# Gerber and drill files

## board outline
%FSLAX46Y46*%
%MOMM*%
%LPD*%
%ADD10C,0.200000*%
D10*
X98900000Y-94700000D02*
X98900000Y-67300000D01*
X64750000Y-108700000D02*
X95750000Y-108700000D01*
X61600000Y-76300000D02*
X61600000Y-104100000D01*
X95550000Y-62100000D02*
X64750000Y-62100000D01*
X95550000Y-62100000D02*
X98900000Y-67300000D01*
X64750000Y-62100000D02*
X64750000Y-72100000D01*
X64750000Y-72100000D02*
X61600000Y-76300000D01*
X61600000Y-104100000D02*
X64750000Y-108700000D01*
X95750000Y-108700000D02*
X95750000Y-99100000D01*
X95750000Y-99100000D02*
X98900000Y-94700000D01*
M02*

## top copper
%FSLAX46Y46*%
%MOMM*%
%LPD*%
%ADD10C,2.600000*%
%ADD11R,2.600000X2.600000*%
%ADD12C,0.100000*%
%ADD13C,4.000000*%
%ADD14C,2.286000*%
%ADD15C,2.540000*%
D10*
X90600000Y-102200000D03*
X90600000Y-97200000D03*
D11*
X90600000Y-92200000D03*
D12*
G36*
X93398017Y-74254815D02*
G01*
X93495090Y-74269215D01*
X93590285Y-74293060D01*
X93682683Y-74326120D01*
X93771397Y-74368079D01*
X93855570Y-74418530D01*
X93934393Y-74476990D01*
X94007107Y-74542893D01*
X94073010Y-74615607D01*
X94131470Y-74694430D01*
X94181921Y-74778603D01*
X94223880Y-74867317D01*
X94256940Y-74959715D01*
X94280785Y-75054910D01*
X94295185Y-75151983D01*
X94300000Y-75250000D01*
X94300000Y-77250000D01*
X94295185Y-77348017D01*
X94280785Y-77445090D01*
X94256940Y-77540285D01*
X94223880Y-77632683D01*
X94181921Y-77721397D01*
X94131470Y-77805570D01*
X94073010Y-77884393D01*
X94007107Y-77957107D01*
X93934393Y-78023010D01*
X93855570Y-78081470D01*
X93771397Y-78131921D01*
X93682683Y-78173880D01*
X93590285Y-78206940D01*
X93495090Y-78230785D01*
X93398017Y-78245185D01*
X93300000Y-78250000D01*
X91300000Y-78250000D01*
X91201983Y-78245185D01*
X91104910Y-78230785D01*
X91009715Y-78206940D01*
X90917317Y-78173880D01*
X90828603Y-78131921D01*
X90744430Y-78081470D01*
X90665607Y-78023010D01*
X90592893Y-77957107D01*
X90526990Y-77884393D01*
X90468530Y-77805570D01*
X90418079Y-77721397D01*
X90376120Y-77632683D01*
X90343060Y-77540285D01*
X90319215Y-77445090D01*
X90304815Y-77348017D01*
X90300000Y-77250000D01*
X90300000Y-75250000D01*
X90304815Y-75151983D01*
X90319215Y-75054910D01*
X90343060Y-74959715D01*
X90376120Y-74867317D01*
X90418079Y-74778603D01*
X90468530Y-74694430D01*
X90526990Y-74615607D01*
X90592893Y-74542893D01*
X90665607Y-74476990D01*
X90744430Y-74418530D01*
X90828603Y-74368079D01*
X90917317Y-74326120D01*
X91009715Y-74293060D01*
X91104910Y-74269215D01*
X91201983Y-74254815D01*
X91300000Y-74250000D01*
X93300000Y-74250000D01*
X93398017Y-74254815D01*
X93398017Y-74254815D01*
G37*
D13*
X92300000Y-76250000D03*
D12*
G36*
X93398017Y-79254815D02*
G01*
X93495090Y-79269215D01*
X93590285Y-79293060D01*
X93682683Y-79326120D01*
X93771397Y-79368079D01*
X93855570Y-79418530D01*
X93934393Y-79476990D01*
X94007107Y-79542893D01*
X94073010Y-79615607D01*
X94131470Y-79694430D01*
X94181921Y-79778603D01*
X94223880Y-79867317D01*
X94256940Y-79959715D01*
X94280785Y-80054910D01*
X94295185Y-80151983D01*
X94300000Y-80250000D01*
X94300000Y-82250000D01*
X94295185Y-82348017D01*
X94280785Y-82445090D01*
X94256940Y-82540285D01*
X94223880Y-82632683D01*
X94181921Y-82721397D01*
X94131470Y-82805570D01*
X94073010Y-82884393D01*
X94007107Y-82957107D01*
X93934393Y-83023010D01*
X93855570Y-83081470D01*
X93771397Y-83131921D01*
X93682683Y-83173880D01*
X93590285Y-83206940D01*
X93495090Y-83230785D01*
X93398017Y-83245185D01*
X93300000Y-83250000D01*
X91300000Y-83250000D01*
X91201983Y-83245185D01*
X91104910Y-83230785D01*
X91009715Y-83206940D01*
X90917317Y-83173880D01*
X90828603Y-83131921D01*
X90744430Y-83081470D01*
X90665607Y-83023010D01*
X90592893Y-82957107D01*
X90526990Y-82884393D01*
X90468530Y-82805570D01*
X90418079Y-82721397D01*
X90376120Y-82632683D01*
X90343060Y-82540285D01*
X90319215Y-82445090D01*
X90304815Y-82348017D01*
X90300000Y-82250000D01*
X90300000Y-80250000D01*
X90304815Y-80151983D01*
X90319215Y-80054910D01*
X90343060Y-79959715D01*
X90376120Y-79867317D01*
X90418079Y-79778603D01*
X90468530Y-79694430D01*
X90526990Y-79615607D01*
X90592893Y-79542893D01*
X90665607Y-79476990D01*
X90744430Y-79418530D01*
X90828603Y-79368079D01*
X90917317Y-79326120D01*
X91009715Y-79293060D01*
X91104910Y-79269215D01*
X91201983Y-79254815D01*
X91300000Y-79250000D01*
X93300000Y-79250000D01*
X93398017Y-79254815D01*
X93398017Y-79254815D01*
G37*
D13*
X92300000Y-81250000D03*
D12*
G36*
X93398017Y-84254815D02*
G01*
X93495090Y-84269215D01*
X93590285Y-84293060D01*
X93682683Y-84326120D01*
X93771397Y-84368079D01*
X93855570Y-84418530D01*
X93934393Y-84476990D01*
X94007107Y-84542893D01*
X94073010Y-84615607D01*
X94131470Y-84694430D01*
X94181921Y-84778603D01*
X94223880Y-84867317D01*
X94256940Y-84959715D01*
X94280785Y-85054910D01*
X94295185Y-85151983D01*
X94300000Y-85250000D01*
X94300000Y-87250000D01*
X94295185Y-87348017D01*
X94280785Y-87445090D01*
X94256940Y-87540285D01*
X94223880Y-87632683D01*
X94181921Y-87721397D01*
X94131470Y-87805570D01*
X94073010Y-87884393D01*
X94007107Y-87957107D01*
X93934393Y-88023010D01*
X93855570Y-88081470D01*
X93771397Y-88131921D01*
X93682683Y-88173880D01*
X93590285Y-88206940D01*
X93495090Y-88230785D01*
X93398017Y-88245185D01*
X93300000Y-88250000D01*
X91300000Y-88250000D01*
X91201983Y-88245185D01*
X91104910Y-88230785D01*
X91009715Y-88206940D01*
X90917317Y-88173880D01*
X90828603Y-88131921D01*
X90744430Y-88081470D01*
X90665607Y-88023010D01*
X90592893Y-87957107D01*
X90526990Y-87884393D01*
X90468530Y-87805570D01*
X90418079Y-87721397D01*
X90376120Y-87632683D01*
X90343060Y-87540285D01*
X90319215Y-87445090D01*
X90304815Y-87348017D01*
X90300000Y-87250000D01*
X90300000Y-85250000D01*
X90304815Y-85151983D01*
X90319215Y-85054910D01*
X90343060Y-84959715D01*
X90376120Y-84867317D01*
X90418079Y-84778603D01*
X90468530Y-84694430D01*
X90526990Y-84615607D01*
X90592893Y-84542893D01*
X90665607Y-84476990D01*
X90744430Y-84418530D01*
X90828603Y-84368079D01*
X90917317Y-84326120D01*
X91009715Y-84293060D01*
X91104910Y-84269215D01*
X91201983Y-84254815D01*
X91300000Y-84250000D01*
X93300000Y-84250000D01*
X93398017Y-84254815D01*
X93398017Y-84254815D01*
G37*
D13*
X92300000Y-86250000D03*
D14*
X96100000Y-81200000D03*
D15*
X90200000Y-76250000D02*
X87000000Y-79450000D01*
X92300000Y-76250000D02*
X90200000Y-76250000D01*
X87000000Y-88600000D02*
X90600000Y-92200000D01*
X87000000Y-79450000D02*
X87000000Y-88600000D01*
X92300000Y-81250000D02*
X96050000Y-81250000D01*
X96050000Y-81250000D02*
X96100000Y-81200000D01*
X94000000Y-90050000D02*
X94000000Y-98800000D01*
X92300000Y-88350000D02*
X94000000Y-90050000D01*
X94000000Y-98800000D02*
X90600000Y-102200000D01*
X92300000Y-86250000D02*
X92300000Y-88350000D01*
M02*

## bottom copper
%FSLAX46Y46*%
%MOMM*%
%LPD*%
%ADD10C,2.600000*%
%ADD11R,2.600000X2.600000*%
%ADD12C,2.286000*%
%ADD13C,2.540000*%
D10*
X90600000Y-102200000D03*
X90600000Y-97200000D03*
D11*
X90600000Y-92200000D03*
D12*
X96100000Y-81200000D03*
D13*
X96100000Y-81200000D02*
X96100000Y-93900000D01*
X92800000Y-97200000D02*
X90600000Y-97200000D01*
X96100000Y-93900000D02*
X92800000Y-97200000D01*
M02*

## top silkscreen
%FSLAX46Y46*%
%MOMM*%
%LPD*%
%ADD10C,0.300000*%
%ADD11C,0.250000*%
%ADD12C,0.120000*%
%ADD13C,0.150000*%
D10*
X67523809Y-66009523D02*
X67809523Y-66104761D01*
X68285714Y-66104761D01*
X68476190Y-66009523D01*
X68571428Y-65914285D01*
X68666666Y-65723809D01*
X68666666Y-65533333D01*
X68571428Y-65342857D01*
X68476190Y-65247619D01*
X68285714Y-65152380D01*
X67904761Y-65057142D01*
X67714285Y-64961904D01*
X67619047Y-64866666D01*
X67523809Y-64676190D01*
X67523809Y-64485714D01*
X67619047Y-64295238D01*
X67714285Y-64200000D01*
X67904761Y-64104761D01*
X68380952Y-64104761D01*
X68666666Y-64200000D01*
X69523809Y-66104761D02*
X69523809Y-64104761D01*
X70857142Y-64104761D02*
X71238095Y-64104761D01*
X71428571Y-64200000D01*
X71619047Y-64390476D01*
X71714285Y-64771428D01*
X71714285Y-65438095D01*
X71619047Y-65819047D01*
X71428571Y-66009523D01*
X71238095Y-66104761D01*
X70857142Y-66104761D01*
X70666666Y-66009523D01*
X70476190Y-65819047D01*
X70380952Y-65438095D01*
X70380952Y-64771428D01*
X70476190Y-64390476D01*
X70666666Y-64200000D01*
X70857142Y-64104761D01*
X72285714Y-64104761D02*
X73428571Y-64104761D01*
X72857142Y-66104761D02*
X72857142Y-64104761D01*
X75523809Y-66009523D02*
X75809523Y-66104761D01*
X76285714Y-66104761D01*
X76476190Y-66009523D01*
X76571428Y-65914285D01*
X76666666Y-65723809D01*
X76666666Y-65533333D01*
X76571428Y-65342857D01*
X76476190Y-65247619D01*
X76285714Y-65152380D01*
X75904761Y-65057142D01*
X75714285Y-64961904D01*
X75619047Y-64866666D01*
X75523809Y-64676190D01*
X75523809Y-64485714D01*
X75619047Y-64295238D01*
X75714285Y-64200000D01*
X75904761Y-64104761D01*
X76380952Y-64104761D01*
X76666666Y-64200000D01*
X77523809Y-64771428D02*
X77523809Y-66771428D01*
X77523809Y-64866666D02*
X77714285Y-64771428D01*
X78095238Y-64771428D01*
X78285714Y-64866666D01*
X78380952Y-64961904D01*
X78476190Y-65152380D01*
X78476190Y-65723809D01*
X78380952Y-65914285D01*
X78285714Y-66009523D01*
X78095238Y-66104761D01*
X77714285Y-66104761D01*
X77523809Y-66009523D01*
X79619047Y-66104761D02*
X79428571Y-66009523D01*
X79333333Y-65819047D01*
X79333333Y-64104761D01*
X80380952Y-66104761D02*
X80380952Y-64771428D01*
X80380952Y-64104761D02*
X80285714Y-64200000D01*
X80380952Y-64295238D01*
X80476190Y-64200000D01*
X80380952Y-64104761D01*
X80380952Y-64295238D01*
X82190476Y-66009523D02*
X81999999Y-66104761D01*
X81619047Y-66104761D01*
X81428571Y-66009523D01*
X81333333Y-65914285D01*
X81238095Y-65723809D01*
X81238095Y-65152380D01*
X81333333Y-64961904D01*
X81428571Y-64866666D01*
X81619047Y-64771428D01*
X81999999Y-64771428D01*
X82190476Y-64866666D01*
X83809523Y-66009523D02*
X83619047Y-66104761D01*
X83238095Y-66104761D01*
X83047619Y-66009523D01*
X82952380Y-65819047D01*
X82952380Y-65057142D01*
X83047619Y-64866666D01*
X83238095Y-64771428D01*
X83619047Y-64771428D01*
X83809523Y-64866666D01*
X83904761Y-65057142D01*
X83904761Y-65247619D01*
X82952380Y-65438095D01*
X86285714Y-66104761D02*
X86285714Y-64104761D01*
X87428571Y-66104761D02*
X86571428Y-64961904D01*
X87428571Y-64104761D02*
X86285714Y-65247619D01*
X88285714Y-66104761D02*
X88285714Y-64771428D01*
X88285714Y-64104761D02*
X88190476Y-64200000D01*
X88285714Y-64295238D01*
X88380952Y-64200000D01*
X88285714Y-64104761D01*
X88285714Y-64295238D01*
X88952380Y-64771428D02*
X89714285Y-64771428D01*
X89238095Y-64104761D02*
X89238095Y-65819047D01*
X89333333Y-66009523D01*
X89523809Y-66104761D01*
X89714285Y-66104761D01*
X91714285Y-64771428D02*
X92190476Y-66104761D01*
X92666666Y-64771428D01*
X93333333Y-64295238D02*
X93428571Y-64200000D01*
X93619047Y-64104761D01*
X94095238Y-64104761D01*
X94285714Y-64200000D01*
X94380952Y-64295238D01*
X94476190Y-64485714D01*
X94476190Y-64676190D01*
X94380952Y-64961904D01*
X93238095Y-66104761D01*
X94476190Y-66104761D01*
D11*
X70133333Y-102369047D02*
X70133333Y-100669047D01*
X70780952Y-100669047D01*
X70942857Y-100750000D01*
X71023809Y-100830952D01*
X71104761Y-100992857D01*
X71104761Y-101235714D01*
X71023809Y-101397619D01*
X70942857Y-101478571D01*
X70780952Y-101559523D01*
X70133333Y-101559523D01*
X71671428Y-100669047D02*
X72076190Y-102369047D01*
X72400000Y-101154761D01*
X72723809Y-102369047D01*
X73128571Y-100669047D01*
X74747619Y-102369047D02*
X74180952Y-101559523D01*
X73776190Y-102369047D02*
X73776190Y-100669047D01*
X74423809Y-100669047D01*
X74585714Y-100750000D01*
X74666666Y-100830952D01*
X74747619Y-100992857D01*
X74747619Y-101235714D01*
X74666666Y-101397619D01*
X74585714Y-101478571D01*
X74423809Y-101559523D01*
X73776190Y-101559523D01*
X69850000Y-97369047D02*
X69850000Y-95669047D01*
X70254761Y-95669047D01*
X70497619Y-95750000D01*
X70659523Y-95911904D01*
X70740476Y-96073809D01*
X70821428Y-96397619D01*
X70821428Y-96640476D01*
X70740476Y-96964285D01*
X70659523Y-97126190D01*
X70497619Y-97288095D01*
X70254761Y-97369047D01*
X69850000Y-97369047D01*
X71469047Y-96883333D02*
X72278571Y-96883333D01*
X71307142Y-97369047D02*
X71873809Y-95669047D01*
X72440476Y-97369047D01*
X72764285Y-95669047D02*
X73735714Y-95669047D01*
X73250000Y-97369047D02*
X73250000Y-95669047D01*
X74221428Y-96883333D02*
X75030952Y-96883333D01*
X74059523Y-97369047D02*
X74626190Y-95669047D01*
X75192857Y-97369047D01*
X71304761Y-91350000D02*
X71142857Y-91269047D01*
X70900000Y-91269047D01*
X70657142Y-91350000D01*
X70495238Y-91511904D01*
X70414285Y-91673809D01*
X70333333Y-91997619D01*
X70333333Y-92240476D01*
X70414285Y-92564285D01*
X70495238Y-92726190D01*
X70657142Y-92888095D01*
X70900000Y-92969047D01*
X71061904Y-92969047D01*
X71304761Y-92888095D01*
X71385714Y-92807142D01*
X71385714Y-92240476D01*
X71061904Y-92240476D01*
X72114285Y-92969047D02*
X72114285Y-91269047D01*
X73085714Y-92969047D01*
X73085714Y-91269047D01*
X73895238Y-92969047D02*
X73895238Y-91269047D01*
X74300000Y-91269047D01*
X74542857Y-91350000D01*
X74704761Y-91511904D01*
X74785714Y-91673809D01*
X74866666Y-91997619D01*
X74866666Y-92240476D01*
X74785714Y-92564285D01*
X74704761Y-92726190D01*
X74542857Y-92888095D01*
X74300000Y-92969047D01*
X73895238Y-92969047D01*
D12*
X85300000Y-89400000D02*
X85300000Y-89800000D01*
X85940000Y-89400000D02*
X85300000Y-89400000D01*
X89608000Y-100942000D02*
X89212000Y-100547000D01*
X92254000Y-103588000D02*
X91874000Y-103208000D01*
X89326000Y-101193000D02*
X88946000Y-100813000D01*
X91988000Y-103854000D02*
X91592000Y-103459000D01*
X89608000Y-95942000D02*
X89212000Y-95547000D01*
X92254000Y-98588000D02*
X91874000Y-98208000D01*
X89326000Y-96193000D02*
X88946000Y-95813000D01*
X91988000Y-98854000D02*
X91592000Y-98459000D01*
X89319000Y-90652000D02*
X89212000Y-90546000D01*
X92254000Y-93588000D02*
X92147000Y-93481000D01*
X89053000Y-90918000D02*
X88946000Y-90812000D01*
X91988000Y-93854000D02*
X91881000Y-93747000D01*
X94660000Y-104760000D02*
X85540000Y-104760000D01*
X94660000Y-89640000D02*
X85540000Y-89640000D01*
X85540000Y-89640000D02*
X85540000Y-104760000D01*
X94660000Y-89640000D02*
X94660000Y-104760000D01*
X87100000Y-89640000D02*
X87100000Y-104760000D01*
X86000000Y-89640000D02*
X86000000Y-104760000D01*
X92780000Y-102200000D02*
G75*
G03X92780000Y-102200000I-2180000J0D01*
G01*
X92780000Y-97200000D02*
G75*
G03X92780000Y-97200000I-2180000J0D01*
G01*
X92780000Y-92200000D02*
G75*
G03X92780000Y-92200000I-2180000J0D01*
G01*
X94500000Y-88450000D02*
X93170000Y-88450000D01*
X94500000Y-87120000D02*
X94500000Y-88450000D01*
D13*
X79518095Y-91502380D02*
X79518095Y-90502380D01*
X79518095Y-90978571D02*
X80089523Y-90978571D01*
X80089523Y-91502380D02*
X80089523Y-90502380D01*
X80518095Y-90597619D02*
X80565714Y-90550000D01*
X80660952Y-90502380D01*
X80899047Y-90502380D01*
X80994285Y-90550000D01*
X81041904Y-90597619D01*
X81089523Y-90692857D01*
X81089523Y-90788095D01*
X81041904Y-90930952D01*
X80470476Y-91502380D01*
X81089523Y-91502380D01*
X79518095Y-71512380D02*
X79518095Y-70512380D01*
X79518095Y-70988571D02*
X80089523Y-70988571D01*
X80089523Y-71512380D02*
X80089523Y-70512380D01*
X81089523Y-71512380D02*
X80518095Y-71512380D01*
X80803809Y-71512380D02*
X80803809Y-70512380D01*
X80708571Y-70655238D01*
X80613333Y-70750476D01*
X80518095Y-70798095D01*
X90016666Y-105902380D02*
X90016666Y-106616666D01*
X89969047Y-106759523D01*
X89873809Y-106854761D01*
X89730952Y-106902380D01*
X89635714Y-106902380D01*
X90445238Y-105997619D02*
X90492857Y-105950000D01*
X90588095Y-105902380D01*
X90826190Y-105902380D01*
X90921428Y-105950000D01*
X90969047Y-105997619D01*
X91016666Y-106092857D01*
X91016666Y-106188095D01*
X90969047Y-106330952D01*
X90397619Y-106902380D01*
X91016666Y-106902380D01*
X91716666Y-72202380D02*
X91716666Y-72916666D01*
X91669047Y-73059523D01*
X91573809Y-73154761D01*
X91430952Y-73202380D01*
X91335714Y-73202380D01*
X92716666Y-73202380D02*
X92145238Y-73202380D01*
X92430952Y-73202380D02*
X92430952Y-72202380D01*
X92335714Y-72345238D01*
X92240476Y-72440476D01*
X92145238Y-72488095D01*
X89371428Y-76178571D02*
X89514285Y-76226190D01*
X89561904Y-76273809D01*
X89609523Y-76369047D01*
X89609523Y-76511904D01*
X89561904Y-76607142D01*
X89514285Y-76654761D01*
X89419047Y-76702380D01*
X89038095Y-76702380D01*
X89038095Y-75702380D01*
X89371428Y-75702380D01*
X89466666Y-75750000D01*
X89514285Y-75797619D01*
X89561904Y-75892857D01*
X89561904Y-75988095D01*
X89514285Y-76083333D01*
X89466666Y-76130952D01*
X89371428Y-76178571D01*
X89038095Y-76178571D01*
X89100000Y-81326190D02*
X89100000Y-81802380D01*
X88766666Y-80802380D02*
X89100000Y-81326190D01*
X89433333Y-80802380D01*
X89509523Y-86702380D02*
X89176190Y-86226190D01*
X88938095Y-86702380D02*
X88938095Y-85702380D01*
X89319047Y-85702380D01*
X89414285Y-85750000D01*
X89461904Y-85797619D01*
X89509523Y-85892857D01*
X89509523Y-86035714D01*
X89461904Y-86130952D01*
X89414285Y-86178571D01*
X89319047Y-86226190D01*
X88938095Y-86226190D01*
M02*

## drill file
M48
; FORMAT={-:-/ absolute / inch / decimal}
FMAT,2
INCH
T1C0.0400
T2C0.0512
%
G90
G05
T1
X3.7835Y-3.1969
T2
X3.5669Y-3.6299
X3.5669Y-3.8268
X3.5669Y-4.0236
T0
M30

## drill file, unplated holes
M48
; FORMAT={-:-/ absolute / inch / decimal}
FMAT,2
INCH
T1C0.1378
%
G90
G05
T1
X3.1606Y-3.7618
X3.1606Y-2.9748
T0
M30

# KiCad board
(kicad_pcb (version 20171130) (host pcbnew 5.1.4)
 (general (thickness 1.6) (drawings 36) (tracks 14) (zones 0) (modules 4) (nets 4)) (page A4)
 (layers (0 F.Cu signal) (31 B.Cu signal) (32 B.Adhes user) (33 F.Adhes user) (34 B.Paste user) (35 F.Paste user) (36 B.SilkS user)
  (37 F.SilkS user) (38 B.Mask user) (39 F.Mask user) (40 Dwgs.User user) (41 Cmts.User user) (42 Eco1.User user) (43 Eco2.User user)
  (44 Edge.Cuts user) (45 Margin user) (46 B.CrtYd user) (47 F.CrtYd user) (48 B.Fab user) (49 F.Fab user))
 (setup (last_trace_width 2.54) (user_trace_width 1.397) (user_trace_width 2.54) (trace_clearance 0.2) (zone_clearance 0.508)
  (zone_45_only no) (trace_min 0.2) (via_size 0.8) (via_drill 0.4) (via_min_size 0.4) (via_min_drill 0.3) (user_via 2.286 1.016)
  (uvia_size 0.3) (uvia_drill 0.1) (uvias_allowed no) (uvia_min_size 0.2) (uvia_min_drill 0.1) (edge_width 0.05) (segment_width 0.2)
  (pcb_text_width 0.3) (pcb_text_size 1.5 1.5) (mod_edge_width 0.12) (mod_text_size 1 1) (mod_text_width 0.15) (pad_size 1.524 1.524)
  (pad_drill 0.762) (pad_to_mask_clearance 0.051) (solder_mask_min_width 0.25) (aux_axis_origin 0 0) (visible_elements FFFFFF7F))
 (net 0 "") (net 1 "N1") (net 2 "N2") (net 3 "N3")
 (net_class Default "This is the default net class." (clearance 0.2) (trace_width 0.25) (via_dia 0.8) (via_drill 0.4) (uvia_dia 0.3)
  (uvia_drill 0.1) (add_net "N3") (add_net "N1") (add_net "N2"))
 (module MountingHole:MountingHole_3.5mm (layer F.Cu) (at 80.28 95.55)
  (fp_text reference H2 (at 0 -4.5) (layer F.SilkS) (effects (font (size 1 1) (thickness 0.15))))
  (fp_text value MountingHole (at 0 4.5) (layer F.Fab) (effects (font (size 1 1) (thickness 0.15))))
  (pad 1 np_thru_hole circle (at 0 0) (size 3.5 3.5) (drill 3.5) (layers *.Cu *.Mask)))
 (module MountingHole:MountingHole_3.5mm (layer F.Cu) (at 80.28 75.56)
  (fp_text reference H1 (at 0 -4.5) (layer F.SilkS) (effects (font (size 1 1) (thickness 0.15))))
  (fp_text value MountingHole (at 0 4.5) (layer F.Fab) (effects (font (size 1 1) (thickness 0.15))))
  (pad 1 np_thru_hole circle (at 0 0) (size 3.5 3.5) (drill 3.5) (layers *.Cu *.Mask)))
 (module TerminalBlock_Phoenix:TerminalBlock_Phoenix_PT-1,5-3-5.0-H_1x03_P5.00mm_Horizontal (layer F.Cu) (at 90.6 92.2 270)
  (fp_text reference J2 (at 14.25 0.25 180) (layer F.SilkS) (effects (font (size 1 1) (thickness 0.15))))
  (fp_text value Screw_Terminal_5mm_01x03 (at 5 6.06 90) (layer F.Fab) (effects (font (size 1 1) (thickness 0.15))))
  (fp_line (start -2.8 5.3) (end -2.4 5.3) (layer F.SilkS) (width 0.12))
  (fp_line (start -2.8 4.66) (end -2.8 5.3) (layer F.SilkS) (width 0.12))
  (fp_line (start 8.742 0.992) (end 8.347 1.388) (layer F.SilkS) (width 0.12))
  (fp_line (start 11.388 -1.654) (end 11.008 -1.274) (layer F.SilkS) (width 0.12))
  (fp_line (start 8.993 1.274) (end 8.613 1.654) (layer F.SilkS) (width 0.12))
  (fp_line (start 11.654 -1.388) (end 11.259 -0.992) (layer F.SilkS) (width 0.12))
  (fp_line (start 3.742 0.992) (end 3.347 1.388) (layer F.SilkS) (width 0.12))
  (fp_line (start 6.388 -1.654) (end 6.008 -1.274) (layer F.SilkS) (width 0.12))
  (fp_line (start 3.993 1.274) (end 3.613 1.654) (layer F.SilkS) (width 0.12))
  (fp_line (start 6.654 -1.388) (end 6.259 -0.992) (layer F.SilkS) (width 0.12))
  (fp_line (start -1.548 1.281) (end -1.654 1.388) (layer F.SilkS) (width 0.12))
  (fp_line (start 1.388 -1.654) (end 1.281 -1.547) (layer F.SilkS) (width 0.12))
  (fp_line (start -1.282 1.547) (end -1.388 1.654) (layer F.SilkS) (width 0.12))
  (fp_line (start 1.654 -1.388) (end 1.547 -1.281) (layer F.SilkS) (width 0.12))
  (fp_line (start 12.56 -4.06) (end 12.56 5.06) (layer F.SilkS) (width 0.12))
  (fp_line (start -2.56 -4.06) (end -2.56 5.06) (layer F.SilkS) (width 0.12))
  (fp_line (start -2.56 5.06) (end 12.56 5.06) (layer F.SilkS) (width 0.12))
  (fp_line (start -2.56 -4.06) (end 12.56 -4.06) (layer F.SilkS) (width 0.12))
  (fp_line (start -2.56 3.5) (end 12.56 3.5) (layer F.SilkS) (width 0.12))
  (fp_line (start -2.56 4.6) (end 12.56 4.6) (layer F.SilkS) (width 0.12))
  (fp_circle (center 10 0) (end 12.18 0) (layer F.SilkS) (width 0.12))
  (fp_circle (center 5 0) (end 7.18 0) (layer F.SilkS) (width 0.12))
  (fp_circle (center 0 0) (end 2.18 0) (layer F.SilkS) (width 0.12))
  (pad 3 thru_hole circle (at 10 0 270) (size 2.6 2.6) (drill 1.3) (layers *.Cu *.Mask) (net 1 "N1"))
  (pad 2 thru_hole circle (at 5 0 270) (size 2.6 2.6) (drill 1.3) (layers *.Cu *.Mask) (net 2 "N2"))
  (pad 1 thru_hole rect (at 0 0 270) (size 2.6 2.6) (drill 1.3) (layers *.Cu *.Mask) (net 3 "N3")))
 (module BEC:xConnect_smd (layer F.Cu) (at 92.3 86.25 180)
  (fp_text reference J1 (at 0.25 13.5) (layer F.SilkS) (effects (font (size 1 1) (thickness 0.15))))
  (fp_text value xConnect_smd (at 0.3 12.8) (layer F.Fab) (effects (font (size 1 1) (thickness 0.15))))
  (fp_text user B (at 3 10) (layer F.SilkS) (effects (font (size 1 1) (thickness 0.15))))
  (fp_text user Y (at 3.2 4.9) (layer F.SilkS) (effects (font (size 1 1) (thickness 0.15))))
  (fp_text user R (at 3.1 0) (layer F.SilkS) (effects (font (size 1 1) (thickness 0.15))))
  (fp_line (start -2.2 -2.2) (end -0.87 -2.2) (layer F.SilkS) (width 0.12))
  (fp_line (start -2.2 -0.87) (end -2.2 -2.2) (layer F.SilkS) (width 0.12))
  (pad B smd roundrect (at 0 10 180) (size 4 4) (layers F.Cu F.Paste F.Mask) (roundrect_rratio 0.25) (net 3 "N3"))
  (pad Y smd roundrect (at 0 5 180) (size 4 4) (layers F.Cu F.Paste F.Mask) (roundrect_rratio 0.25) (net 2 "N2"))
  (pad R smd roundrect (at 0 0 180) (size 4 4) (layers F.Cu F.Paste F.Mask) (roundrect_rratio 0.25) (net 1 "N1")))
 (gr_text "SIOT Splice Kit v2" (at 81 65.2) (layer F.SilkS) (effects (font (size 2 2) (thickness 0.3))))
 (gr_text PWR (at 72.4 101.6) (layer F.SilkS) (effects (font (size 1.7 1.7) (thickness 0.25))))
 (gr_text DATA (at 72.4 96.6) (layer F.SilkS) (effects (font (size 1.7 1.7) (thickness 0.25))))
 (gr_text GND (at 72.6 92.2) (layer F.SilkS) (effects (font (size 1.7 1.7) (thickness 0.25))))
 (gr_line (start 98.9 94.7) (end 98.9 67.3) (layer Edge.Cuts) (width 0.2))
 (gr_line (start 64.75 108.7) (end 95.75 108.7) (layer Edge.Cuts) (width 0.2))
 (gr_line (start 61.6 76.3) (end 61.6 104.1) (layer Edge.Cuts) (width 0.2))
 (gr_line (start 95.55 62.1) (end 64.75 62.1) (layer Edge.Cuts) (width 0.2))
 (gr_line (start 95.55 62.1) (end 98.9 67.3) (layer Edge.Cuts) (width 0.2))
 (gr_line (start 64.75 62.1) (end 64.75 72.1) (layer Edge.Cuts) (width 0.2))
 (gr_line (start 64.75 72.1) (end 61.6 76.3) (layer Edge.Cuts) (width 0.2))
 (gr_line (start 61.6 104.1) (end 64.75 108.7) (layer Edge.Cuts) (width 0.2))
 (gr_line (start 95.75 108.7) (end 95.75 99.1) (layer Edge.Cuts) (width 0.2))
 (gr_line (start 95.75 99.1) (end 98.9 94.7) (layer Edge.Cuts) (width 0.2))
 (segment (start 90.2 76.25) (end 87 79.45) (width 2.54) (layer F.Cu) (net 3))
 (segment (start 92.3 76.25) (end 90.2 76.25) (width 2.54) (layer F.Cu) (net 3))
 (segment (start 87 88.6) (end 90.6 92.2) (width 2.54) (layer F.Cu) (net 3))
 (segment (start 87 79.45) (end 87 88.6) (width 2.54) (layer F.Cu) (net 3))
 (via (at 96.1 81.2) (size 2.286) (drill 1.016) (layers F.Cu B.Cu) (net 2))
 (segment (start 92.3 81.25) (end 96.05 81.25) (width 2.54) (layer F.Cu) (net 2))
 (segment (start 96.05 81.25) (end 96.1 81.2) (width 2.54) (layer F.Cu) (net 2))
 (segment (start 96.1 81.2) (end 96.1 93.9) (width 2.54) (layer B.Cu) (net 2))
 (segment (start 92.8 97.2) (end 90.6 97.2) (width 2.54) (layer B.Cu) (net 2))
 (segment (start 96.1 93.9) (end 92.8 97.2) (width 2.54) (layer B.Cu) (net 2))
 (segment (start 94 90.05) (end 94 98.8) (width 2.54) (layer F.Cu) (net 1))
 (segment (start 92.3 88.35) (end 94 90.05) (width 2.54) (layer F.Cu) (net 1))
 (segment (start 94 98.8) (end 90.6 102.2) (width 2.54) (layer F.Cu) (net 1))
 (segment (start 92.3 86.25) (end 92.3 88.35) (width 2.54) (layer F.Cu) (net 1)))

